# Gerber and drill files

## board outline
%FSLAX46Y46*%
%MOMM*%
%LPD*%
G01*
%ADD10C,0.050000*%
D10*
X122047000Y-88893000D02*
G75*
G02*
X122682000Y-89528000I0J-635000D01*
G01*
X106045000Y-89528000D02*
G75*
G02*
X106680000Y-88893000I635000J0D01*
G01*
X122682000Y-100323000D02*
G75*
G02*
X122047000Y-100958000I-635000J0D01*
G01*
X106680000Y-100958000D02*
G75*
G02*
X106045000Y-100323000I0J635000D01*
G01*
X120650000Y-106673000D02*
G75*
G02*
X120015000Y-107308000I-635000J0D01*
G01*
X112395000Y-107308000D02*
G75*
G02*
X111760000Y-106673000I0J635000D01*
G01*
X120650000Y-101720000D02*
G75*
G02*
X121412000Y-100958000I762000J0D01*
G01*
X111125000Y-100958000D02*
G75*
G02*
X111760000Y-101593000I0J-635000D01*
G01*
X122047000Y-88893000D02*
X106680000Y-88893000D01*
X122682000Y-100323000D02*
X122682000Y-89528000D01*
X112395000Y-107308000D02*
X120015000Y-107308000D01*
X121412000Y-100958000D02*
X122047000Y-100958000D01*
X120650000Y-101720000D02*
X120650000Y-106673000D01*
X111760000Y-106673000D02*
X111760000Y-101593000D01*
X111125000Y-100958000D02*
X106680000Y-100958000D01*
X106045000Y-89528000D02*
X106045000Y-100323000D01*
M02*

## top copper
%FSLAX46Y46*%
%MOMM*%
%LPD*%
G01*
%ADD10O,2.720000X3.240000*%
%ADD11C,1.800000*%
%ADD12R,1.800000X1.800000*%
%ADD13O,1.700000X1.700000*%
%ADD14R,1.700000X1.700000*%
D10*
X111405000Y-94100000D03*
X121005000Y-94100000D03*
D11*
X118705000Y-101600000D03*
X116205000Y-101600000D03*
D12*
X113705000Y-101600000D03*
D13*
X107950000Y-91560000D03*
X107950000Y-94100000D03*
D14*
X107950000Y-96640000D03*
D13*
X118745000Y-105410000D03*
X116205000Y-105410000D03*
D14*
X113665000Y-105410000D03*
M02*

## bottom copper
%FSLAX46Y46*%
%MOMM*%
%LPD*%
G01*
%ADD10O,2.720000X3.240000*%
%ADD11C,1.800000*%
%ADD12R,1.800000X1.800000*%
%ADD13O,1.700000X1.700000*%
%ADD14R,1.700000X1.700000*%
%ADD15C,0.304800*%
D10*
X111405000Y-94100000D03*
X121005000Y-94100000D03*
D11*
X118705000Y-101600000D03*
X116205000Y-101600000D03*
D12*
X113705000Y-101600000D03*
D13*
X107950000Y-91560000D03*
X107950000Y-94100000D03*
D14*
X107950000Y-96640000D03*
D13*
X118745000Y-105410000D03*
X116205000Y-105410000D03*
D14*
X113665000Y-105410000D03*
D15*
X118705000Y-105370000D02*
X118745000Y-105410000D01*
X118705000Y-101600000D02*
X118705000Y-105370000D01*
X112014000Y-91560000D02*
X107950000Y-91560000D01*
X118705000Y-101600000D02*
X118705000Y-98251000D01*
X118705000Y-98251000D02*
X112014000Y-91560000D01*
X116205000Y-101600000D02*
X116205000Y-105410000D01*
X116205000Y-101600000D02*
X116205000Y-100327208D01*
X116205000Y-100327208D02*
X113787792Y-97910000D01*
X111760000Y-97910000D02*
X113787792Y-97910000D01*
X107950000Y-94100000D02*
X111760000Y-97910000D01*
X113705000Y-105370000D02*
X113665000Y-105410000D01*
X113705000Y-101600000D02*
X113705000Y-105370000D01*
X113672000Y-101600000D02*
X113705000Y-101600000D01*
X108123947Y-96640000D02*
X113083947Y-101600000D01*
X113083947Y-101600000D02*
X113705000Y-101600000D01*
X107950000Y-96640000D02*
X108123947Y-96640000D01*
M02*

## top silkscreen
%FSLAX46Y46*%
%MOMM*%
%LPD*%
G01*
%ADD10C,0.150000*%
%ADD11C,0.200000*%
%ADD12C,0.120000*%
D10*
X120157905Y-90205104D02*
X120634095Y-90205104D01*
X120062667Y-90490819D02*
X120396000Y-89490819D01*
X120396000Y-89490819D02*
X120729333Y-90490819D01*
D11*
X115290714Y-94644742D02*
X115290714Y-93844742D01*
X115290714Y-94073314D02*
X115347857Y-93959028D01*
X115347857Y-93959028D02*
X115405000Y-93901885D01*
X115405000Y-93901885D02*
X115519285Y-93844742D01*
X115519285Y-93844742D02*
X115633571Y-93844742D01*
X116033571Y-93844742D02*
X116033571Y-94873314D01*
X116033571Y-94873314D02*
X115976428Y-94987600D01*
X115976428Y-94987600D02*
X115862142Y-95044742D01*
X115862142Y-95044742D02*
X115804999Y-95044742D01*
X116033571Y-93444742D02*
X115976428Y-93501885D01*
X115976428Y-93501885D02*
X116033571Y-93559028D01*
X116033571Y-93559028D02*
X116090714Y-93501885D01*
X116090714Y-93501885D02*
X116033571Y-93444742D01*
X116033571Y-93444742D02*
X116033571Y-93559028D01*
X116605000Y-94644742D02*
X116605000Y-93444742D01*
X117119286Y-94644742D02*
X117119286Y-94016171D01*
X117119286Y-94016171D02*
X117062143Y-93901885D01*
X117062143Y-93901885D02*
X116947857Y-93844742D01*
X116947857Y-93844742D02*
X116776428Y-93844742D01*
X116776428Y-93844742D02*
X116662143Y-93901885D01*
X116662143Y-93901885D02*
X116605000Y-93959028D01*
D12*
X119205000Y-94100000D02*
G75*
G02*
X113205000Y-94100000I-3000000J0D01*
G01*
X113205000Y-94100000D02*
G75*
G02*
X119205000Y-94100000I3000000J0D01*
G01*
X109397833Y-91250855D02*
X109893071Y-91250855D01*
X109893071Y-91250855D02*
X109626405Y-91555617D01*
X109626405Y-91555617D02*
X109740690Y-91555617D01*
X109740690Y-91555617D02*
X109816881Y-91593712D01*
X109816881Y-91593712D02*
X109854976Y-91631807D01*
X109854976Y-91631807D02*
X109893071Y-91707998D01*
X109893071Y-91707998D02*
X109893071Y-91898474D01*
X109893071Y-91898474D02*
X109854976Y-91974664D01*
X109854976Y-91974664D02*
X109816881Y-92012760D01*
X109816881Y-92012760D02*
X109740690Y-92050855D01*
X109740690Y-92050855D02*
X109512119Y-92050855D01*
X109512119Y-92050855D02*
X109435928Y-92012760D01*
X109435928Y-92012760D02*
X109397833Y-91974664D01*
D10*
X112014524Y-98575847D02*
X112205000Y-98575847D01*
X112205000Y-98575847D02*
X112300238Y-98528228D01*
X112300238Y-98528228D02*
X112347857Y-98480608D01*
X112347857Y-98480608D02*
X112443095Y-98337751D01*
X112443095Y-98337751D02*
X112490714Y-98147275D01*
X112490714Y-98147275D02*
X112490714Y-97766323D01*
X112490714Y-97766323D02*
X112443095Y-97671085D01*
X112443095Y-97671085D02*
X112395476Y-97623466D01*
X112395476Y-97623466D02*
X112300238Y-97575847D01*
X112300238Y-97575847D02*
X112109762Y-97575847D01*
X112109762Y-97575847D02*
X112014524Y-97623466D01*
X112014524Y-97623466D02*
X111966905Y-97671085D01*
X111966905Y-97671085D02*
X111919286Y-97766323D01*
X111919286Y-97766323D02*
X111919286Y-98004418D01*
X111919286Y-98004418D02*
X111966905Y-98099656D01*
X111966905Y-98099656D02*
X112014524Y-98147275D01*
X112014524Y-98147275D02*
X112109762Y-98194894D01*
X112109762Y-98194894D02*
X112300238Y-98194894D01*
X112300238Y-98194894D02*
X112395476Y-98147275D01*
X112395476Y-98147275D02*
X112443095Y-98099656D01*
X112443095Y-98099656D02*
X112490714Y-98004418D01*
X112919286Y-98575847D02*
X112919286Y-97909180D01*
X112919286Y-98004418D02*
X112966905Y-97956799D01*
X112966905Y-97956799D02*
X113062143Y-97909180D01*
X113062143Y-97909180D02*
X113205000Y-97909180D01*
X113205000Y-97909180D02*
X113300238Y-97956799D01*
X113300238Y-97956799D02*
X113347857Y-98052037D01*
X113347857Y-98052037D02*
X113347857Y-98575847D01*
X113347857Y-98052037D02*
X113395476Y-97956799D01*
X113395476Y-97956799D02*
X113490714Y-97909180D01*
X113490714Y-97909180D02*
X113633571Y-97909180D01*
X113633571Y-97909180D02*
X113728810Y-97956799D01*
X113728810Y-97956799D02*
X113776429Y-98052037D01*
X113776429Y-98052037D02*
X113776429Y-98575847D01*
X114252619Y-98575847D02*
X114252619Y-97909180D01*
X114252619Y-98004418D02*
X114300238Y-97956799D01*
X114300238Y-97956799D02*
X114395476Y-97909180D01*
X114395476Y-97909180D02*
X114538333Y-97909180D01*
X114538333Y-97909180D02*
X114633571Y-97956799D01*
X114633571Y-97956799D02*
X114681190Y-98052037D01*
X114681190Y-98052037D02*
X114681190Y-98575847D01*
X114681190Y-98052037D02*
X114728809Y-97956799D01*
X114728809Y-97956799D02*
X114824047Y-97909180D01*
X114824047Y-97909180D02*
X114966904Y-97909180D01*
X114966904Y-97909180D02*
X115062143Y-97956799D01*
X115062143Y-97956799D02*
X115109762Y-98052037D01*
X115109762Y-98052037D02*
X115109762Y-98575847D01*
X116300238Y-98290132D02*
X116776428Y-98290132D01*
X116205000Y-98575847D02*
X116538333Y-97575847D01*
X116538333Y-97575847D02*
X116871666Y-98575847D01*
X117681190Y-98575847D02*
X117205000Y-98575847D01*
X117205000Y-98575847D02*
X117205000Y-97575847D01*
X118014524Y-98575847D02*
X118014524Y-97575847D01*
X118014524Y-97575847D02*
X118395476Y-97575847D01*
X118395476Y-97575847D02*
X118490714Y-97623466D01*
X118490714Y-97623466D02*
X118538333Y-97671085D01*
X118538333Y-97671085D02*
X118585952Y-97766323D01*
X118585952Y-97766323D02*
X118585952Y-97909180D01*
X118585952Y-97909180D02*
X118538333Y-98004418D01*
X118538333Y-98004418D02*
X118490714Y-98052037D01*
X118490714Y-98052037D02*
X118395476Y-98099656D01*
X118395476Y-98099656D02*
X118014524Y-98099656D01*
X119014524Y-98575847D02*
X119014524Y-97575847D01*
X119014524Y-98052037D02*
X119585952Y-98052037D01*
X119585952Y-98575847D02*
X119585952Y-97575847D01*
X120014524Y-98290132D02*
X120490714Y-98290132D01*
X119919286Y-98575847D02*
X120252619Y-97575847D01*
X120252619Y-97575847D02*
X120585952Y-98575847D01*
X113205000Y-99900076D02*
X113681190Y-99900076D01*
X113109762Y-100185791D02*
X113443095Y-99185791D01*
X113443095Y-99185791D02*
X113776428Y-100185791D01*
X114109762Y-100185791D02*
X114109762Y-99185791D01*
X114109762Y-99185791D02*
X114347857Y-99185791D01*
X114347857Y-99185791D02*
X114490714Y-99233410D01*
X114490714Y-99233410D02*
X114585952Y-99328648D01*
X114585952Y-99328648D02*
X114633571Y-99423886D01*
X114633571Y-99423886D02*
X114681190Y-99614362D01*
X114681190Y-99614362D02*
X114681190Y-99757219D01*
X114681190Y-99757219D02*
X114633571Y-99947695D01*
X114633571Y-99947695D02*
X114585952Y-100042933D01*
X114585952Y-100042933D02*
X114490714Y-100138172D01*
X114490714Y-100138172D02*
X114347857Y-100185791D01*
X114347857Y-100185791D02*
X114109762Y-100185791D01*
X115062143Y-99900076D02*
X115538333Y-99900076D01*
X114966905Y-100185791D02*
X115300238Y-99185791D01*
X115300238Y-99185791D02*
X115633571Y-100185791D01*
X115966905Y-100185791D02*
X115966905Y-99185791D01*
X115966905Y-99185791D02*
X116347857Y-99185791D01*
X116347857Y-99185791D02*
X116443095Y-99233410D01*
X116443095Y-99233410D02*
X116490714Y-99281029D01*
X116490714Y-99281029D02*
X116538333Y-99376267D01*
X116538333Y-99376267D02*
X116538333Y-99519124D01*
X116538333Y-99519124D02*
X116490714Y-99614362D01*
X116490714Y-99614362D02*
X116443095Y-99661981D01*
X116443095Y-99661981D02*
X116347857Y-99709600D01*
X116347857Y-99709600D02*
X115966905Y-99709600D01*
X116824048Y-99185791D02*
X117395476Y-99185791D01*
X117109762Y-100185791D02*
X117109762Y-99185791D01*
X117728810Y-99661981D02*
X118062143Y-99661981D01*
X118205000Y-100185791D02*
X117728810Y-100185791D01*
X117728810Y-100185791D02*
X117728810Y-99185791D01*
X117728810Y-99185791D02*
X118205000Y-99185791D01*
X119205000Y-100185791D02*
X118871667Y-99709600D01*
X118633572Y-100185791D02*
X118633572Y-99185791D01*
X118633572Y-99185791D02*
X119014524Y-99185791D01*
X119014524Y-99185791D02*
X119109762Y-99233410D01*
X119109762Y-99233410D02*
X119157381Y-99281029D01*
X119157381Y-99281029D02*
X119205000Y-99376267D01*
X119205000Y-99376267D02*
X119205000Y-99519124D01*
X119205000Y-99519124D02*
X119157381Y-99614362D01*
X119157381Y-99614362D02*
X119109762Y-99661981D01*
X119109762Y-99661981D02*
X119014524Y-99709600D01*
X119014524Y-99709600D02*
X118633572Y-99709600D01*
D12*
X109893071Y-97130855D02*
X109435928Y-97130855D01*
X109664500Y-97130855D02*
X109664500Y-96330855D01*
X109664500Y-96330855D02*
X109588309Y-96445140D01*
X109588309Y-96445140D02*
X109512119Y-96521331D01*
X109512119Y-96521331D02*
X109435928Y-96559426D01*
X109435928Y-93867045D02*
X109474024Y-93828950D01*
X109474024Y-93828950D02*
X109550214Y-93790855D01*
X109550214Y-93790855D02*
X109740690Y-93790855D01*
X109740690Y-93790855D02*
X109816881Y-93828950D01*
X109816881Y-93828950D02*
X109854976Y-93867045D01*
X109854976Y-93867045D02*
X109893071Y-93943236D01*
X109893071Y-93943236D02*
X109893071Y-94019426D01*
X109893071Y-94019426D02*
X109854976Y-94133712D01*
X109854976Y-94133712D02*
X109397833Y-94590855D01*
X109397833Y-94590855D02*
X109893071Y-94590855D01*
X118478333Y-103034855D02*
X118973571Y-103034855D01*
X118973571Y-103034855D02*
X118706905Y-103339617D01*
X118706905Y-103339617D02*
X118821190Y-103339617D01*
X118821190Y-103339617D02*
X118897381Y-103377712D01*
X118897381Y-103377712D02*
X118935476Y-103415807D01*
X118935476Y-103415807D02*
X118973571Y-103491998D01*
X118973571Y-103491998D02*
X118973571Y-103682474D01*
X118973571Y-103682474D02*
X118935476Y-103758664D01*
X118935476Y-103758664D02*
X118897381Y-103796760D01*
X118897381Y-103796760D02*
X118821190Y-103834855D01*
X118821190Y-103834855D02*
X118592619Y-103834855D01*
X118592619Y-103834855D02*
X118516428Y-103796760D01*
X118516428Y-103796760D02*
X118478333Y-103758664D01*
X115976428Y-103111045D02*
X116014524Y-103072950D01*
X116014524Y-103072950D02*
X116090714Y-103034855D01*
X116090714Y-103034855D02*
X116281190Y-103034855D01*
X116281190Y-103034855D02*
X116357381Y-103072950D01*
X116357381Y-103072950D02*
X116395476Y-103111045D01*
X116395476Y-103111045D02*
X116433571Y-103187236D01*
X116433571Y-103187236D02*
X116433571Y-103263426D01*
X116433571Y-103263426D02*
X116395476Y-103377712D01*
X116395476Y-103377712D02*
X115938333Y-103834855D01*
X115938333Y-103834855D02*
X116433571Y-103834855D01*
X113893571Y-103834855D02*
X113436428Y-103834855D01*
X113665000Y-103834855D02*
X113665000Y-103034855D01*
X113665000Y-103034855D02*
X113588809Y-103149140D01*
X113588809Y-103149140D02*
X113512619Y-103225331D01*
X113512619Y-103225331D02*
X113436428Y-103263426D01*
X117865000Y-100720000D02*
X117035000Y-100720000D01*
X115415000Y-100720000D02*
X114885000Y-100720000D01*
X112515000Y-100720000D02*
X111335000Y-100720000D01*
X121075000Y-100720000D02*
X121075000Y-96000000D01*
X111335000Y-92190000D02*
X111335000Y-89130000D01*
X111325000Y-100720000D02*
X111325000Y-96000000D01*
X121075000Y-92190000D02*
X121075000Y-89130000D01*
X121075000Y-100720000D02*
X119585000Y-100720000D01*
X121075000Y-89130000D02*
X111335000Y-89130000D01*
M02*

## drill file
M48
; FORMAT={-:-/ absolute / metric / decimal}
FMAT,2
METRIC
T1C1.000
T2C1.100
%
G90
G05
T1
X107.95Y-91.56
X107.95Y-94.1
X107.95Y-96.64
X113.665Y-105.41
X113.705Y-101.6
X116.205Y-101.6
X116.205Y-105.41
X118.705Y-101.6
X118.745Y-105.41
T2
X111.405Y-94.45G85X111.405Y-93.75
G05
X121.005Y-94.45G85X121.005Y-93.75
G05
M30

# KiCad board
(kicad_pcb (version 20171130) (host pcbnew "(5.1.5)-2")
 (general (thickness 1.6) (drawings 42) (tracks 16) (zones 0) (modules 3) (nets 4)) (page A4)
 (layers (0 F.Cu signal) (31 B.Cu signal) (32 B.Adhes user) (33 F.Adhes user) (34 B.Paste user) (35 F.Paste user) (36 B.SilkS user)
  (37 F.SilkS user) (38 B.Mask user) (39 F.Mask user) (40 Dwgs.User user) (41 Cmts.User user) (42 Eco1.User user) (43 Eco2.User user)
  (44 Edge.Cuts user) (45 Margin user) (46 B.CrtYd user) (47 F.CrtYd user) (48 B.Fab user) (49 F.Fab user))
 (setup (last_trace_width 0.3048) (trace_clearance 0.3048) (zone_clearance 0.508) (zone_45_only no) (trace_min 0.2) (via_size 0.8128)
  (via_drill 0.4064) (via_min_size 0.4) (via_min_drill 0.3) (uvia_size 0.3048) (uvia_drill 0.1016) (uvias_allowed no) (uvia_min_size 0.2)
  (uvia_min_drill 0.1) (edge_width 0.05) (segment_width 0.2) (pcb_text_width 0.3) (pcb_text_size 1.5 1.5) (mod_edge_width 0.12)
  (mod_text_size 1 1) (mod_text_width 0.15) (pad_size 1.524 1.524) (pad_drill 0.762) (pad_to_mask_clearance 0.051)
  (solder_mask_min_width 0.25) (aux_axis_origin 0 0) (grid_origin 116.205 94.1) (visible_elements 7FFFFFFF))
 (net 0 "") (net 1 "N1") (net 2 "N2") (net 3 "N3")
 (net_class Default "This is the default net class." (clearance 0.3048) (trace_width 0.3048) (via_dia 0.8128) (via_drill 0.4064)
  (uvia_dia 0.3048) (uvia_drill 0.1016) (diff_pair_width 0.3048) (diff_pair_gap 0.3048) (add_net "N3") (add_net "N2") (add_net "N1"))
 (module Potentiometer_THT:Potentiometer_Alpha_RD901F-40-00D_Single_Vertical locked (layer F.Cu) (at 113.705 101.6 90)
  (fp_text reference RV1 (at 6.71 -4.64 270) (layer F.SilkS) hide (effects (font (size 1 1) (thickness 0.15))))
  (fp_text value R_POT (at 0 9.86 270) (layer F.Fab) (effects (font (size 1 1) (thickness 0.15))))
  (fp_line (start 0.88 4.16) (end 0.88 3.33) (layer F.SilkS) (width 0.12))
  (fp_line (start 0.88 1.71) (end 0.88 1.18) (layer F.SilkS) (width 0.12))
  (fp_line (start 0.88 -1.19) (end 0.88 -2.37) (layer F.SilkS) (width 0.12))
  (fp_line (start 0.88 7.37) (end 5.6 7.37) (layer F.SilkS) (width 0.12))
  (fp_line (start 9.41 -2.37) (end 12.47 -2.37) (layer F.SilkS) (width 0.12))
  (fp_line (start 0.88 -2.38) (end 5.6 -2.38) (layer F.SilkS) (width 0.12))
  (fp_line (start 9.41 7.37) (end 12.47 7.37) (layer F.SilkS) (width 0.12))
  (fp_line (start 0.88 7.37) (end 0.88 5.88) (layer F.SilkS) (width 0.12))
  (fp_line (start 12.47 7.37) (end 12.47 -2.37) (layer F.SilkS) (width 0.12))
  (pad "" thru_hole oval (at 7.5 -2.3 180) (size 2.72 3.24) (drill oval 1.1 1.8) (layers *.Cu *.Mask))
  (pad "" thru_hole oval (at 7.5 7.3 180) (size 2.72 3.24) (drill oval 1.1 1.8) (layers *.Cu *.Mask))
  (pad 3 thru_hole circle (at 0 5 180) (size 1.8 1.8) (drill 1) (layers *.Cu *.Mask) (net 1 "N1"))
  (pad 2 thru_hole circle (at 0 2.5 180) (size 1.8 1.8) (drill 1) (layers *.Cu *.Mask) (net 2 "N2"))
  (pad 1 thru_hole rect (at 0 0 180) (size 1.8 1.8) (drill 1) (layers *.Cu *.Mask) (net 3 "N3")))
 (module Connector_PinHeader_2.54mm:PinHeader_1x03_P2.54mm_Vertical (layer B.Cu) (at 107.95 96.64)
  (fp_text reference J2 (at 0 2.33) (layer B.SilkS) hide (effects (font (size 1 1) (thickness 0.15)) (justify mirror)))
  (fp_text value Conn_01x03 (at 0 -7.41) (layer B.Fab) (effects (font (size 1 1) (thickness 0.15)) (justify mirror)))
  (pad 3 thru_hole oval (at 0 -5.08) (size 1.7 1.7) (drill 1) (layers *.Cu *.Mask) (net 1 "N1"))
  (pad 2 thru_hole oval (at 0 -2.54) (size 1.7 1.7) (drill 1) (layers *.Cu *.Mask) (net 2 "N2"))
  (pad 1 thru_hole rect (at 0 0) (size 1.7 1.7) (drill 1) (layers *.Cu *.Mask) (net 3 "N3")))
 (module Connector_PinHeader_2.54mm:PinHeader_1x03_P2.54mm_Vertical (layer B.Cu) (at 113.665 105.41 270)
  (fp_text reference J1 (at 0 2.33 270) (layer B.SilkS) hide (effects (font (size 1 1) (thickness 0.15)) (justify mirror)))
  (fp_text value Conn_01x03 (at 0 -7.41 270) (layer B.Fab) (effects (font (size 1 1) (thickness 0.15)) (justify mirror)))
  (pad 3 thru_hole oval (at 0 -5.08 270) (size 1.7 1.7) (drill 1) (layers *.Cu *.Mask) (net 1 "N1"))
  (pad 2 thru_hole oval (at 0 -2.54 270) (size 1.7 1.7) (drill 1) (layers *.Cu *.Mask) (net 2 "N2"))
  (pad 1 thru_hole rect (at 0 0 270) (size 1.7 1.7) (drill 1) (layers *.Cu *.Mask) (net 3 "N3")))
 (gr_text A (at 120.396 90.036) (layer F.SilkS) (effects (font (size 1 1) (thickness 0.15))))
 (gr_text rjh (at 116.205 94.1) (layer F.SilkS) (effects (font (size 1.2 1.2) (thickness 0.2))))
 (gr_arc (start 122.047 89.528) (end 122.682 89.528) (angle -90) (layer Edge.Cuts) (width 0.05))
 (gr_arc (start 106.68 89.528) (end 106.68 88.893) (angle -90) (layer Edge.Cuts) (width 0.05))
 (gr_arc (start 122.047 100.323) (end 122.047 100.958) (angle -90) (layer Edge.Cuts) (width 0.05))
 (gr_arc (start 106.68 100.323) (end 106.045 100.323) (angle -90) (layer Edge.Cuts) (width 0.05))
 (gr_arc (start 120.015 106.673) (end 120.015 107.308) (angle -90) (layer Edge.Cuts) (width 0.05))
 (gr_arc (start 112.395 106.673) (end 111.76 106.673) (angle -90) (layer Edge.Cuts) (width 0.05))
 (gr_arc (start 121.412 101.72) (end 121.412 100.958) (angle -90) (layer Edge.Cuts) (width 0.05))
 (gr_arc (start 111.125 101.593) (end 111.76 101.593) (angle -90) (layer Edge.Cuts) (width 0.05))
 (gr_circle (center 116.205 94.1) (end 119.205 94.1) (layer F.SilkS) (width 0.12))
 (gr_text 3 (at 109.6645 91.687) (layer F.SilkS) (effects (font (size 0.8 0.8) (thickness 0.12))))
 (gr_line (start 122.047 88.893) (end 106.68 88.893) (layer Edge.Cuts) (width 0.05))
 (gr_line (start 122.682 100.323) (end 122.682 89.528) (layer Edge.Cuts) (width 0.05))
 (gr_line (start 112.395 107.308) (end 120.015 107.308) (layer Edge.Cuts) (width 0.05))
 (gr_line (start 121.412 100.958) (end 122.047 100.958) (layer Edge.Cuts) (width 0.05))
 (gr_line (start 120.65 101.72) (end 120.65 106.673) (layer Edge.Cuts) (width 0.05))
 (gr_line (start 111.76 106.673) (end 111.76 101.593) (layer Edge.Cuts) (width 0.05))
 (gr_line (start 111.125 100.958) (end 106.68 100.958) (layer Edge.Cuts) (width 0.05))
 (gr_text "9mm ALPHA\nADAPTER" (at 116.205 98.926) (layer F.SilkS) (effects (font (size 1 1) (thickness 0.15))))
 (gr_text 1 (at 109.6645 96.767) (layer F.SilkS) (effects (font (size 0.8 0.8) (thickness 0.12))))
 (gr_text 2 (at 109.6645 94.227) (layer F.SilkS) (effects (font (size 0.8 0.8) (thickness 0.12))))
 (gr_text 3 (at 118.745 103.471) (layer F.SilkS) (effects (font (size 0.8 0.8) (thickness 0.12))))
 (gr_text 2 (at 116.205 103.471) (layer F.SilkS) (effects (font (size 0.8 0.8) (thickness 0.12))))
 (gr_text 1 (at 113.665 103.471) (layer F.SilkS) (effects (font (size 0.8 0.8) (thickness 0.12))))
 (gr_line (start 106.045 89.528) (end 106.045 100.323) (layer Edge.Cuts) (width 0.05))
 (segment (start 118.705 105.37) (end 118.745 105.41) (width 0.3048) (layer B.Cu) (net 1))
 (segment (start 118.705 101.6) (end 118.705 105.37) (width 0.3048) (layer B.Cu) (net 1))
 (segment (start 112.014 91.56) (end 107.95 91.56) (width 0.3048) (layer B.Cu) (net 1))
 (segment (start 118.705 101.6) (end 118.705 98.251) (width 0.3048) (layer B.Cu) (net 1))
 (segment (start 118.705 98.251) (end 112.014 91.56) (width 0.3048) (layer B.Cu) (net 1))
 (segment (start 116.205 101.6) (end 116.205 105.41) (width 0.3048) (layer B.Cu) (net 2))
 (segment (start 116.205 101.6) (end 116.205 100.327208) (width 0.3048) (layer B.Cu) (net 2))
 (segment (start 116.205 100.327208) (end 113.787792 97.91) (width 0.3048) (layer B.Cu) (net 2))
 (segment (start 111.76 97.91) (end 113.787792 97.91) (width 0.3048) (layer B.Cu) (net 2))
 (segment (start 107.95 94.1) (end 111.76 97.91) (width 0.3048) (layer B.Cu) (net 2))
 (segment (start 113.705 105.37) (end 113.665 105.41) (width 0.3048) (layer B.Cu) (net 3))
 (segment (start 113.705 101.6) (end 113.705 105.37) (width 0.3048) (layer B.Cu) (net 3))
 (segment (start 113.672 101.6) (end 113.705 101.6) (width 0.3048) (layer B.Cu) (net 3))
 (segment (start 108.123947 96.64) (end 113.083947 101.6) (width 0.3048) (layer B.Cu) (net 3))
 (segment (start 113.083947 101.6) (end 113.705 101.6) (width 0.3048) (layer B.Cu) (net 3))
 (segment (start 107.95 96.64) (end 108.123947 96.64) (width 0.3048) (layer B.Cu) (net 3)))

